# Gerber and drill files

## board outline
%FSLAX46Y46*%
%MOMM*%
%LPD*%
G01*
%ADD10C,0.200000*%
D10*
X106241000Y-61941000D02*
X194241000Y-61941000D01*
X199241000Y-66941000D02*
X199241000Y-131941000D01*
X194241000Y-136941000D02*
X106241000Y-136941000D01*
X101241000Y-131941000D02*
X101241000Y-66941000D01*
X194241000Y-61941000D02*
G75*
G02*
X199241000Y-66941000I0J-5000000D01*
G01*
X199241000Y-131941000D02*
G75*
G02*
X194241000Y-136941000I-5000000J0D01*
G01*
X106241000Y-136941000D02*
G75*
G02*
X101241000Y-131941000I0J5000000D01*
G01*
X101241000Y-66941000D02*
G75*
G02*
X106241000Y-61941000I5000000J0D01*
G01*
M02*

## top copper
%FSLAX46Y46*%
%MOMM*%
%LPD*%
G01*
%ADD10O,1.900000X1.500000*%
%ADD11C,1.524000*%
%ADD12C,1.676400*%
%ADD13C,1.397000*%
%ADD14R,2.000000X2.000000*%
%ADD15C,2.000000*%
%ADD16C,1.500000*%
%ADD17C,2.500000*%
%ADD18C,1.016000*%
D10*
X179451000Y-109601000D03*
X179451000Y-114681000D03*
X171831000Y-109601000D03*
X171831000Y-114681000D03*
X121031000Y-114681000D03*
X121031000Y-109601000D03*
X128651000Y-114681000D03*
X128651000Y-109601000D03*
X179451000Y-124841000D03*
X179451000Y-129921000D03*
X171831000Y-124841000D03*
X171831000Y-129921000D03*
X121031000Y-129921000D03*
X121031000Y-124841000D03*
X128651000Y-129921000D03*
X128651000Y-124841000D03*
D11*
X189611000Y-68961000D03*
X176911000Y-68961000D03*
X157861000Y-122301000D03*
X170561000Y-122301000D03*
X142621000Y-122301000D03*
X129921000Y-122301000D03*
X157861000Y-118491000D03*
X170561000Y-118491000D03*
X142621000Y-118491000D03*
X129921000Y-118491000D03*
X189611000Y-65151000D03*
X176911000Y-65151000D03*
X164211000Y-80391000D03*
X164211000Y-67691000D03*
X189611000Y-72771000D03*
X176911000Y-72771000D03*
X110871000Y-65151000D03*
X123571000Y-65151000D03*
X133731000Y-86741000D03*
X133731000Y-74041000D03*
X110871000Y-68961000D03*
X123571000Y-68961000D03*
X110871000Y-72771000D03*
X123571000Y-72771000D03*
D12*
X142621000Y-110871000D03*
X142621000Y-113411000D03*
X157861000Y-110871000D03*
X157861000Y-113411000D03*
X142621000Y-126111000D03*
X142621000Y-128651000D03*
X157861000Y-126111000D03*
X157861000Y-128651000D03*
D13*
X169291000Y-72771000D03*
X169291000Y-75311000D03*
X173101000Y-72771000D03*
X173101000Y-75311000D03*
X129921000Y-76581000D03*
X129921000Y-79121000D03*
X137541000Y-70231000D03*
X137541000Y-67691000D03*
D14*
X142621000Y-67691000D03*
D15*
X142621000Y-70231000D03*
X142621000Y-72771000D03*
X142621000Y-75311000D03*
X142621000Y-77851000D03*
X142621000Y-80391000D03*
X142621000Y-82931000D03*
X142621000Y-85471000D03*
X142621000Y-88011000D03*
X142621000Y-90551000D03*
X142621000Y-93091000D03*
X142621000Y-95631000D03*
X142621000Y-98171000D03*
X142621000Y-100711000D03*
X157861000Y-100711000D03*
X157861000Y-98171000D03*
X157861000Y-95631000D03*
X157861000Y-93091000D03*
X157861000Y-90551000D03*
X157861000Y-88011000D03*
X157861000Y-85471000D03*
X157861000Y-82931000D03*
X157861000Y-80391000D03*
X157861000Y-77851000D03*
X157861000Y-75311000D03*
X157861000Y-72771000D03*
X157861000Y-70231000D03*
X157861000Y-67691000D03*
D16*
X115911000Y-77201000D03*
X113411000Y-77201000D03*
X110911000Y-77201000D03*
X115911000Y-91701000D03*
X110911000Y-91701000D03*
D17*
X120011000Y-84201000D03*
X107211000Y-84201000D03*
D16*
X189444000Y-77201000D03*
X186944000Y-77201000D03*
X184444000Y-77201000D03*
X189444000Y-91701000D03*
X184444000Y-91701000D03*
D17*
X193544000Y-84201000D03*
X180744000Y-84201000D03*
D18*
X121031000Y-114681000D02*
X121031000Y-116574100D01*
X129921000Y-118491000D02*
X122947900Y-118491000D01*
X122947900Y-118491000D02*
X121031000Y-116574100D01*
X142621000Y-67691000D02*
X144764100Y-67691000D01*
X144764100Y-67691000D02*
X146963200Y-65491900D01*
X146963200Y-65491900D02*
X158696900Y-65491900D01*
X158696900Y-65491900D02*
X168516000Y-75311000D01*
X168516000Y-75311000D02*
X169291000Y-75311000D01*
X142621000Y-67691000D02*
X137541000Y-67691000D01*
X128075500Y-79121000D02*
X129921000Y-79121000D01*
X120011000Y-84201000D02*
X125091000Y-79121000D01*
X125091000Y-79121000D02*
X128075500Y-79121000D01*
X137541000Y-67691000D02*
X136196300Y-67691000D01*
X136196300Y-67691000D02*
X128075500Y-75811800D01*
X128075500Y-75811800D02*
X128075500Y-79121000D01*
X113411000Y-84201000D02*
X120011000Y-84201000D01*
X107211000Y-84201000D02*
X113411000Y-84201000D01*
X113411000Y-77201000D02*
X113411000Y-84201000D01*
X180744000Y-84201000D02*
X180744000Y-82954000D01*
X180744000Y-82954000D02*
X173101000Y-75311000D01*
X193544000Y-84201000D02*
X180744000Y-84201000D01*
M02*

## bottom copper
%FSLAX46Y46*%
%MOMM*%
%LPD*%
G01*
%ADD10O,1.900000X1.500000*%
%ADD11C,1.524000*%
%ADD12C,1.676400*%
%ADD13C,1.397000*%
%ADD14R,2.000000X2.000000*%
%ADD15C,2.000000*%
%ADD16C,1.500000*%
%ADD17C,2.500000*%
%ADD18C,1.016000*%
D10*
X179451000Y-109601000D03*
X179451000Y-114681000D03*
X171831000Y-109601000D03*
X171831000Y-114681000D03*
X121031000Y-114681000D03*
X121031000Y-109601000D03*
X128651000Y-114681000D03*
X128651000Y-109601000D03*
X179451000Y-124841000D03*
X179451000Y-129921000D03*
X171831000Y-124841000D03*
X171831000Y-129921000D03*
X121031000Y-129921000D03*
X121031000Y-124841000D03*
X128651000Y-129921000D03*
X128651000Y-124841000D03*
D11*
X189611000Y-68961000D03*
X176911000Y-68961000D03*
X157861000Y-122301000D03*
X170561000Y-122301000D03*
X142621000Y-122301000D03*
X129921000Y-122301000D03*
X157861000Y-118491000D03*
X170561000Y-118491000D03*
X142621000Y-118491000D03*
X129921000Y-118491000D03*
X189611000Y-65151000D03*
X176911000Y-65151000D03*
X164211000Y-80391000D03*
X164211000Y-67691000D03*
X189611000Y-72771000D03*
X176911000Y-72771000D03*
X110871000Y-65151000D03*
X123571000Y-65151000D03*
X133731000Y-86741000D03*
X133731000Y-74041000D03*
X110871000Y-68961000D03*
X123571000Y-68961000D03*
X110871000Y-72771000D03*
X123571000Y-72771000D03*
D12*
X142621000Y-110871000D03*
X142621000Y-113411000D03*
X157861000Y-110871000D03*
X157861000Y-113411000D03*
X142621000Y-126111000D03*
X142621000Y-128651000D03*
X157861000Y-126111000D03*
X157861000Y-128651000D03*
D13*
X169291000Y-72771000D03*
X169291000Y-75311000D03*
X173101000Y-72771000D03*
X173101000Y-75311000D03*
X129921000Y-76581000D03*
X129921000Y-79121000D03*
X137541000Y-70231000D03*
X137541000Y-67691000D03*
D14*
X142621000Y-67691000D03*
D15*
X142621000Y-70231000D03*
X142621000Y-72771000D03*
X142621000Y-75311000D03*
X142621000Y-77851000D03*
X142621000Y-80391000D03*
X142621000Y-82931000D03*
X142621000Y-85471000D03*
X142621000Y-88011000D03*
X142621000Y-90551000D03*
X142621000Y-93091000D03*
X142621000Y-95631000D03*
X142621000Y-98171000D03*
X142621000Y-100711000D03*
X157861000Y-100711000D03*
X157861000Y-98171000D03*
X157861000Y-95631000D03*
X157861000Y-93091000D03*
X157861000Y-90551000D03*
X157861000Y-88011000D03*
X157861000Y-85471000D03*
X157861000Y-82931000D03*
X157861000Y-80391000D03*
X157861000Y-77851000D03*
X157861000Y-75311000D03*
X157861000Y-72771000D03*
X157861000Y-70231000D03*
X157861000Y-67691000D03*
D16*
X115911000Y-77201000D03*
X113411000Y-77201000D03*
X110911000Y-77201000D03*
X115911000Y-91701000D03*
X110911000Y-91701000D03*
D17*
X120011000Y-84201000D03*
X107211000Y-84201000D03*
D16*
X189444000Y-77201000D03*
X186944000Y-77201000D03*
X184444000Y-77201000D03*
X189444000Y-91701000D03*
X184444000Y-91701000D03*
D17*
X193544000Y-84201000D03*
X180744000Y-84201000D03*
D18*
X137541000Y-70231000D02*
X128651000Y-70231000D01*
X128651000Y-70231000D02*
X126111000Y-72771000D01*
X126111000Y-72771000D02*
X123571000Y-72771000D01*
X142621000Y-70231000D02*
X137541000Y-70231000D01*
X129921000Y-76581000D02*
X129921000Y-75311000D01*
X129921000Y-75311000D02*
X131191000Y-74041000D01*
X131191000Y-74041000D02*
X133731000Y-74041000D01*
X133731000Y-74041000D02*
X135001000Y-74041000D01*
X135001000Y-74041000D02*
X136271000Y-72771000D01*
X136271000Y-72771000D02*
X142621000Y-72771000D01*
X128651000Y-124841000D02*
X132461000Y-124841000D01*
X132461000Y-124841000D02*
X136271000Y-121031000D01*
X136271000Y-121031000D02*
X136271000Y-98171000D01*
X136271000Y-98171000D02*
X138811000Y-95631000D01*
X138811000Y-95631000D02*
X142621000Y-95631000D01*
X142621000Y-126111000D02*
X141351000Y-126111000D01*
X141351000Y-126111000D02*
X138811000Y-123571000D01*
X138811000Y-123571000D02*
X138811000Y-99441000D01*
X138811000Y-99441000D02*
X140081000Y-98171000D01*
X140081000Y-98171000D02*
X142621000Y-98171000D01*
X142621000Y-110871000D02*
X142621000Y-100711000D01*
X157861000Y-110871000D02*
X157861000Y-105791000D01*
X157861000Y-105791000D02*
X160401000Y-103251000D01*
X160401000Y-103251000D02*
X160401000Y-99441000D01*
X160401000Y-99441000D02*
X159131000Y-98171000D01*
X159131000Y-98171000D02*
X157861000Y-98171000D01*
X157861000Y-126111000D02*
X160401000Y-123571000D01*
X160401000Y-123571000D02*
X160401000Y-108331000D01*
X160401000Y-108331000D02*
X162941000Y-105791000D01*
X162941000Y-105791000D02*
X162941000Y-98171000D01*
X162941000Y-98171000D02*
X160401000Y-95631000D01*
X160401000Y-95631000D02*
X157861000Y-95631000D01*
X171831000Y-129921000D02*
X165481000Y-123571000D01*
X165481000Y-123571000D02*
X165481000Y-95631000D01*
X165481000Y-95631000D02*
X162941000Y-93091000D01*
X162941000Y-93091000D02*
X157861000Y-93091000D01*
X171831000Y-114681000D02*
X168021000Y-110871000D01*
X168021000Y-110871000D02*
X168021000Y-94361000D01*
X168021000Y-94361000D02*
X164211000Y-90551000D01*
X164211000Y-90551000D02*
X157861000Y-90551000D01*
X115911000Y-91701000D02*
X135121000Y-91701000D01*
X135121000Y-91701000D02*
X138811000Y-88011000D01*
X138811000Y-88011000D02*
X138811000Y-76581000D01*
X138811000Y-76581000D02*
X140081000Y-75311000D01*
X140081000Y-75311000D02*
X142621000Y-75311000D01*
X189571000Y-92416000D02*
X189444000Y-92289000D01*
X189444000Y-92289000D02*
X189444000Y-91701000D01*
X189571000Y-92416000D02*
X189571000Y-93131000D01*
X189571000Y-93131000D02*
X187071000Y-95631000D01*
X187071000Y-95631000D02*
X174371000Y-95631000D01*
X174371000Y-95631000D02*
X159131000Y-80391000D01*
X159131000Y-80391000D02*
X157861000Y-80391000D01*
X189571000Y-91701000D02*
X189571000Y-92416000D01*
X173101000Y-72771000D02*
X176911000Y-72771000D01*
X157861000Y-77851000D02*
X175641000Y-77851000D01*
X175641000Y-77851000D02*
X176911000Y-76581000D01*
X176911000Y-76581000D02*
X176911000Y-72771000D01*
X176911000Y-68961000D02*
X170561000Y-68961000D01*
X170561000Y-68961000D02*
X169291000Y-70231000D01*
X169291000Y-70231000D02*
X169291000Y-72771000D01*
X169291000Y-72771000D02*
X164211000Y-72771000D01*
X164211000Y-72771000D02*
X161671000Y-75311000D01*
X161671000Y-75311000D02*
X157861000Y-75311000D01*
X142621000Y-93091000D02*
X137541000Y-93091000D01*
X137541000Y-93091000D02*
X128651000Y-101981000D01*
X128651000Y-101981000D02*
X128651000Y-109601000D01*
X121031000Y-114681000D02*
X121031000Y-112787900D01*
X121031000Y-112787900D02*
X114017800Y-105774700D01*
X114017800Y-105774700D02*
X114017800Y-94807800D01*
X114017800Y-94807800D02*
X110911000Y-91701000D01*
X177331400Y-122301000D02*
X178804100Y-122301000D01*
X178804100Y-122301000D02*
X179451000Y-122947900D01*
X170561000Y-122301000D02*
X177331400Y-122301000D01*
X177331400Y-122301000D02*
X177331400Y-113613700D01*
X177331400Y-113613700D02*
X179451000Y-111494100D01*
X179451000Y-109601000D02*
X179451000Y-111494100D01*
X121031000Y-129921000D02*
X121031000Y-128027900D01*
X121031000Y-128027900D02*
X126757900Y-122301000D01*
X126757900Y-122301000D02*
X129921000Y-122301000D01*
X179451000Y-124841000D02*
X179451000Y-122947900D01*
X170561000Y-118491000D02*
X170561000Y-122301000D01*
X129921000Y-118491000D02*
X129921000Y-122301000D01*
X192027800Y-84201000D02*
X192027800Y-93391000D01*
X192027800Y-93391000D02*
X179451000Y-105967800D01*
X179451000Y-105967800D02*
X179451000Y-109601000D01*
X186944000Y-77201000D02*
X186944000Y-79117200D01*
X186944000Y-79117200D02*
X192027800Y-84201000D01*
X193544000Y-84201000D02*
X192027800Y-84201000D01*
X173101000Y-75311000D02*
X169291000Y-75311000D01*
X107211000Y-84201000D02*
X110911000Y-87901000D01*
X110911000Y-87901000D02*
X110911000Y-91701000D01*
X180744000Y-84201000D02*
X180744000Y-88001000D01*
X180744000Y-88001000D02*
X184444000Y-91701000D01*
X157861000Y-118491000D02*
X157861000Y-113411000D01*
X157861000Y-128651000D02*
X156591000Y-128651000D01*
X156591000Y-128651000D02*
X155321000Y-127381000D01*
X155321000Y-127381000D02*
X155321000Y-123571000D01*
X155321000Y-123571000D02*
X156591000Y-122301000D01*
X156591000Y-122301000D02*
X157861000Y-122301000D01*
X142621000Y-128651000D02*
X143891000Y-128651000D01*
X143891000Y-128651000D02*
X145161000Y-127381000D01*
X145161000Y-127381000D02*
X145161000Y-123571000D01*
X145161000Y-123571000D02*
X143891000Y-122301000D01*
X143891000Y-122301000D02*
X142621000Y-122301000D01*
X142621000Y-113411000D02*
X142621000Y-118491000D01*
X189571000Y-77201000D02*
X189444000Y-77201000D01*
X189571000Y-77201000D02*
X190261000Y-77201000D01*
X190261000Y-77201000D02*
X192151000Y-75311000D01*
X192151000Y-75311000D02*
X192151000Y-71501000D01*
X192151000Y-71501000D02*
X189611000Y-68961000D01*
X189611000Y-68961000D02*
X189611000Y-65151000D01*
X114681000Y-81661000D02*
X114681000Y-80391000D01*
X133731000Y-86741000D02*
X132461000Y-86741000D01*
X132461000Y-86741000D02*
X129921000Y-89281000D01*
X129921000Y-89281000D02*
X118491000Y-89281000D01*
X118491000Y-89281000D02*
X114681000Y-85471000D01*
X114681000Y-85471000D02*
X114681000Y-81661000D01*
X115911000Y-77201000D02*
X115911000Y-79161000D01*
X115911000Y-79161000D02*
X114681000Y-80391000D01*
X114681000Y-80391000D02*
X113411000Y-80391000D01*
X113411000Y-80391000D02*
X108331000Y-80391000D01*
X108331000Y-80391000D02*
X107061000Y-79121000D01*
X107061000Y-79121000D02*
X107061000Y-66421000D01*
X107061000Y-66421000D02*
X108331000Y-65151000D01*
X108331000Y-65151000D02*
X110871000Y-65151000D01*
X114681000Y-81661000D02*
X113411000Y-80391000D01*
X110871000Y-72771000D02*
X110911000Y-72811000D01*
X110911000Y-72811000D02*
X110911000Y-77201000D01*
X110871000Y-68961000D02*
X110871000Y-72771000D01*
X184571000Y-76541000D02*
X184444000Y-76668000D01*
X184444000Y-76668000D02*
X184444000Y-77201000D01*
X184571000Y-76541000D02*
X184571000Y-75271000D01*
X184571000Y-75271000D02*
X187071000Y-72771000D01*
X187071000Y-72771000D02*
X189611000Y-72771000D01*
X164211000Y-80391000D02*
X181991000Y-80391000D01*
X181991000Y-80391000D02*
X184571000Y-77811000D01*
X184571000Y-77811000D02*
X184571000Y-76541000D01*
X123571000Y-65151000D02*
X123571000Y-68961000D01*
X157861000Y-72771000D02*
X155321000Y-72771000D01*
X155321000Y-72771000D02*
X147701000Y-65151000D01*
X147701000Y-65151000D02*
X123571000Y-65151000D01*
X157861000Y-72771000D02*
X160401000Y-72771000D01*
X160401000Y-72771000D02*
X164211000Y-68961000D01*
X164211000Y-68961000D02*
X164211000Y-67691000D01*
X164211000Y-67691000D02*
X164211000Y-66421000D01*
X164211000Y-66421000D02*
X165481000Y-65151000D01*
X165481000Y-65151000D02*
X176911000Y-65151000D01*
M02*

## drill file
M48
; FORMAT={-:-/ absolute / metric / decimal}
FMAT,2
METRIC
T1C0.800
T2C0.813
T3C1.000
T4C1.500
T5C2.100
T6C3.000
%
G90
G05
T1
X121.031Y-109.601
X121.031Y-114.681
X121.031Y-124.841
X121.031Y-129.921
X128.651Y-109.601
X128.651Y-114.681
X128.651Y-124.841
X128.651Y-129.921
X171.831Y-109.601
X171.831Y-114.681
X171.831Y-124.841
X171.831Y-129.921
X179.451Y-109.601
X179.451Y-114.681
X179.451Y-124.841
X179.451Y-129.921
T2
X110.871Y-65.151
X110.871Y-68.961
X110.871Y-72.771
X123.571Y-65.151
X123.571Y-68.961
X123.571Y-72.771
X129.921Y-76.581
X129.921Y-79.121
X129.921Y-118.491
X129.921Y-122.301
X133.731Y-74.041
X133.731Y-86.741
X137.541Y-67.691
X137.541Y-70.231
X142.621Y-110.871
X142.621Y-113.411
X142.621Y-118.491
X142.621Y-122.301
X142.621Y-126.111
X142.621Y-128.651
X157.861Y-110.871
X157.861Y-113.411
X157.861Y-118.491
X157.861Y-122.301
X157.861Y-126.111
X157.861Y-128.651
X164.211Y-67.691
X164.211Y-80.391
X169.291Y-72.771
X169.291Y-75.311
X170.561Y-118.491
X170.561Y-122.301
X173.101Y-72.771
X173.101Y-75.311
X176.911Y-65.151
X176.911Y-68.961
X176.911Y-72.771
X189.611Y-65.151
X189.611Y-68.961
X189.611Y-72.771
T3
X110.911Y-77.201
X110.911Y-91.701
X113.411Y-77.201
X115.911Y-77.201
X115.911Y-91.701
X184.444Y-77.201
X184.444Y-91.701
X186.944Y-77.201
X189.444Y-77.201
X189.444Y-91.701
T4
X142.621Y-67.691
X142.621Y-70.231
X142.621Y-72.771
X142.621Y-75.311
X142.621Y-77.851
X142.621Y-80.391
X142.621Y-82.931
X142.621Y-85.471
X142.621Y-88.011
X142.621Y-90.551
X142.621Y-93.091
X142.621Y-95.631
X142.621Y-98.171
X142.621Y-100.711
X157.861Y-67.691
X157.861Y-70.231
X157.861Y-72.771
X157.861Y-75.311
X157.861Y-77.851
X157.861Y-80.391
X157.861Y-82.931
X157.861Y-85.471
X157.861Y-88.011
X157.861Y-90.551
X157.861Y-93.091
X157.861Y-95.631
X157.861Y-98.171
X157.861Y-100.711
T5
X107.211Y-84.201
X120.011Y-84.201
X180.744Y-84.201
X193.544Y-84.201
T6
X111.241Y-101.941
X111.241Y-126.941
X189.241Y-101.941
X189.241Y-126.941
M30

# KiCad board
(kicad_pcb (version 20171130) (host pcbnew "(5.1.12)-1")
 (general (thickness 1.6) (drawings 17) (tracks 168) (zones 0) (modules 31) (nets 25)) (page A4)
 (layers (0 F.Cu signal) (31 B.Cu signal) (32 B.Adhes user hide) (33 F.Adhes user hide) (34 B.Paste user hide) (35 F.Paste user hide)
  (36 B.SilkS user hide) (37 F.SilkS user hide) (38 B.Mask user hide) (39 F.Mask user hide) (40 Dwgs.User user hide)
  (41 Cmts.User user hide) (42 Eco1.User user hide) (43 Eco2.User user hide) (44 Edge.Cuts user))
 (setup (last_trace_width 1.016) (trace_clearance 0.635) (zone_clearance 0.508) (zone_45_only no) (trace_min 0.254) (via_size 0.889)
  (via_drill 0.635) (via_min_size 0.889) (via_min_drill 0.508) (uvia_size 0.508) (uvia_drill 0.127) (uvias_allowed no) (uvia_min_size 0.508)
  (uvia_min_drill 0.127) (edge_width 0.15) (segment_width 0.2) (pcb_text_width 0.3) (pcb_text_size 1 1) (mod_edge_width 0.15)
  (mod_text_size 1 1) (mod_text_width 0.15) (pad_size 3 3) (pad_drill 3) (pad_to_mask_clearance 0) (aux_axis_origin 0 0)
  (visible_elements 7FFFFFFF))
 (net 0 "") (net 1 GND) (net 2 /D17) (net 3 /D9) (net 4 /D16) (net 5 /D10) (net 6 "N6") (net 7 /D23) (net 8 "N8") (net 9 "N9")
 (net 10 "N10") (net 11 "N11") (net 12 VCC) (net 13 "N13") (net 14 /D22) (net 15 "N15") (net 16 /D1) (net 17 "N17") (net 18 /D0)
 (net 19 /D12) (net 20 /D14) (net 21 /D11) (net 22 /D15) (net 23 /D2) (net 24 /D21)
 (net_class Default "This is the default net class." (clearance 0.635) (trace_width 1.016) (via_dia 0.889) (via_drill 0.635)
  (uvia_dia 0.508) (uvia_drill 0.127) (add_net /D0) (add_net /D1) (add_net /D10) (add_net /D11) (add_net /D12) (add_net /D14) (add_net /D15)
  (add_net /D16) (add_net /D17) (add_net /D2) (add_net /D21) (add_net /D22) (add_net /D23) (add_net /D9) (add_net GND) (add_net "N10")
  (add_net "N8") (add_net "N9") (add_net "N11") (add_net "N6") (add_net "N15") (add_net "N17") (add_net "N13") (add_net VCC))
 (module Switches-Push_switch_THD (layer F.Cu) (at 175.641 112.141 180)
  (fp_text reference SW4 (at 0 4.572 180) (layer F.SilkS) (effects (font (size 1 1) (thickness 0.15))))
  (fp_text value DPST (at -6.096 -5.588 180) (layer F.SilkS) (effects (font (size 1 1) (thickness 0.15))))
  (pad 2 thru_hole oval (at -3.81 2.54 180) (size 1.9 1.5) (drill 0.8) (layers *.Cu *.Mask F.SilkS) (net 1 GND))
  (pad 1 thru_hole oval (at -3.81 -2.54 180) (size 1.9 1.5) (drill 0.8) (layers *.Cu *.Mask F.SilkS))
  (pad 4 thru_hole oval (at 3.81 2.54 180) (size 1.9 1.5) (drill 0.8) (layers *.Cu *.Mask F.SilkS))
  (pad 3 thru_hole oval (at 3.81 -2.54 180) (size 1.9 1.5) (drill 0.8) (layers *.Cu *.Mask F.SilkS) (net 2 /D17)))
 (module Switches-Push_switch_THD (layer F.Cu) (at 124.841 112.141)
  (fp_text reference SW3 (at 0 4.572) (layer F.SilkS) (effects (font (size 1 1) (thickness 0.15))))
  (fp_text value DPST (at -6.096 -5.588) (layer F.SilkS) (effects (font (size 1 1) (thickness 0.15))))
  (pad 2 thru_hole oval (at -3.81 2.54) (size 1.9 1.5) (drill 0.8) (layers *.Cu *.Mask F.SilkS) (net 1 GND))
  (pad 1 thru_hole oval (at -3.81 -2.54) (size 1.9 1.5) (drill 0.8) (layers *.Cu *.Mask F.SilkS))
  (pad 4 thru_hole oval (at 3.81 2.54) (size 1.9 1.5) (drill 0.8) (layers *.Cu *.Mask F.SilkS))
  (pad 3 thru_hole oval (at 3.81 -2.54) (size 1.9 1.5) (drill 0.8) (layers *.Cu *.Mask F.SilkS) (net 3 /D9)))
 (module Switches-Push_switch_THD (layer F.Cu) (at 175.641 127.381 180)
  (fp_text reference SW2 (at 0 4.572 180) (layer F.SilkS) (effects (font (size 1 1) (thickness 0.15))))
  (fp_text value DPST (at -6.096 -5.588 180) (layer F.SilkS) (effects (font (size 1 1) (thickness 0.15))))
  (pad 2 thru_hole oval (at -3.81 2.54 180) (size 1.9 1.5) (drill 0.8) (layers *.Cu *.Mask F.SilkS) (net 1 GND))
  (pad 1 thru_hole oval (at -3.81 -2.54 180) (size 1.9 1.5) (drill 0.8) (layers *.Cu *.Mask F.SilkS))
  (pad 4 thru_hole oval (at 3.81 2.54 180) (size 1.9 1.5) (drill 0.8) (layers *.Cu *.Mask F.SilkS))
  (pad 3 thru_hole oval (at 3.81 -2.54 180) (size 1.9 1.5) (drill 0.8) (layers *.Cu *.Mask F.SilkS) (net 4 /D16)))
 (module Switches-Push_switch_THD (layer F.Cu) (at 124.841 127.381)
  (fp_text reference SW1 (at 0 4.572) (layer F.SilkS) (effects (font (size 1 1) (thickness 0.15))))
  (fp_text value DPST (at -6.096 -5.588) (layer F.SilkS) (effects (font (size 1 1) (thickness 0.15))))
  (pad 2 thru_hole oval (at -3.81 2.54) (size 1.9 1.5) (drill 0.8) (layers *.Cu *.Mask F.SilkS) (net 1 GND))
  (pad 1 thru_hole oval (at -3.81 -2.54) (size 1.9 1.5) (drill 0.8) (layers *.Cu *.Mask F.SilkS))
  (pad 4 thru_hole oval (at 3.81 2.54) (size 1.9 1.5) (drill 0.8) (layers *.Cu *.Mask F.SilkS))
  (pad 3 thru_hole oval (at 3.81 -2.54) (size 1.9 1.5) (drill 0.8) (layers *.Cu *.Mask F.SilkS) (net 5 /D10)))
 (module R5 (layer F.Cu) (at 183.261 68.961 180) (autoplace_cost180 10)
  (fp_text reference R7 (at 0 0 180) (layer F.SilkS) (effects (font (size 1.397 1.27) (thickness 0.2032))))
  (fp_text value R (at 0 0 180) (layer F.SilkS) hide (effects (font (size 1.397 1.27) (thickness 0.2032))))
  (pad 1 thru_hole circle (at -6.35 0 180) (size 1.524 1.524) (drill 0.8128) (layers *.Cu *.Mask F.SilkS) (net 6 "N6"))
  (pad 2 thru_hole circle (at 6.35 0 180) (size 1.524 1.524) (drill 0.8128) (layers *.Cu *.Mask F.SilkS) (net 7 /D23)))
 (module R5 (layer F.Cu) (at 164.211 122.301) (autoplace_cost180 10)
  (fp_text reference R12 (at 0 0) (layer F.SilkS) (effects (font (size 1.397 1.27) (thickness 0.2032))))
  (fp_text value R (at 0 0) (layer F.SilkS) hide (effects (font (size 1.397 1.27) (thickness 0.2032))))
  (pad 1 thru_hole circle (at -6.35 0) (size 1.524 1.524) (drill 0.8128) (layers *.Cu *.Mask F.SilkS) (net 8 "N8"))
  (pad 2 thru_hole circle (at 6.35 0) (size 1.524 1.524) (drill 0.8128) (layers *.Cu *.Mask F.SilkS) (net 1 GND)))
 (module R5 (layer F.Cu) (at 136.271 122.301 180) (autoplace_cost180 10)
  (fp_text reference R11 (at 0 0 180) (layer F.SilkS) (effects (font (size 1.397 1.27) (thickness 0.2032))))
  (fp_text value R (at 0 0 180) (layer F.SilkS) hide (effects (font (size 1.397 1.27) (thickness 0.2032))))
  (pad 1 thru_hole circle (at -6.35 0 180) (size 1.524 1.524) (drill 0.8128) (layers *.Cu *.Mask F.SilkS) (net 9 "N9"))
  (pad 2 thru_hole circle (at 6.35 0 180) (size 1.524 1.524) (drill 0.8128) (layers *.Cu *.Mask F.SilkS) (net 1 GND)))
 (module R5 (layer F.Cu) (at 164.211 118.491) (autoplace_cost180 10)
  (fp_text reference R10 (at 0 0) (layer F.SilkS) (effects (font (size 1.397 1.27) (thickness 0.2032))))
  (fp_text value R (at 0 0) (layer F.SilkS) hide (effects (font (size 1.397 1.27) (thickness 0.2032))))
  (pad 1 thru_hole circle (at -6.35 0) (size 1.524 1.524) (drill 0.8128) (layers *.Cu *.Mask F.SilkS) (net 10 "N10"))
  (pad 2 thru_hole circle (at 6.35 0) (size 1.524 1.524) (drill 0.8128) (layers *.Cu *.Mask F.SilkS) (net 1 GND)))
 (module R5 (layer F.Cu) (at 136.271 118.491 180) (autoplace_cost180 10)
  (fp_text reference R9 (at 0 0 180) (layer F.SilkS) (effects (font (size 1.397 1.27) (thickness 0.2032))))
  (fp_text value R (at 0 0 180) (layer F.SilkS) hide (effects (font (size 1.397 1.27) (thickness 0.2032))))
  (pad 1 thru_hole circle (at -6.35 0 180) (size 1.524 1.524) (drill 0.8128) (layers *.Cu *.Mask F.SilkS) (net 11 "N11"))
  (pad 2 thru_hole circle (at 6.35 0 180) (size 1.524 1.524) (drill 0.8128) (layers *.Cu *.Mask F.SilkS) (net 1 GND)))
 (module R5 (layer F.Cu) (at 183.261 65.151 180) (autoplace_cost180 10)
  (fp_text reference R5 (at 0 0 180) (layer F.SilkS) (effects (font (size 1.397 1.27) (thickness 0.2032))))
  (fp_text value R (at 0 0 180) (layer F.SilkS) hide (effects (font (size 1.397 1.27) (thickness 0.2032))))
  (pad 1 thru_hole circle (at -6.35 0 180) (size 1.524 1.524) (drill 0.8128) (layers *.Cu *.Mask F.SilkS) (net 6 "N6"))
  (pad 2 thru_hole circle (at 6.35 0 180) (size 1.524 1.524) (drill 0.8128) (layers *.Cu *.Mask F.SilkS) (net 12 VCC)))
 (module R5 (layer F.Cu) (at 164.211 74.041 90) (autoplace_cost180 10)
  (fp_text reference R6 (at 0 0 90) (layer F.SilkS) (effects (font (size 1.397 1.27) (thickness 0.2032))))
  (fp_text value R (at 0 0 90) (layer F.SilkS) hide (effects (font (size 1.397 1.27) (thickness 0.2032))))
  (pad 1 thru_hole circle (at -6.35 0 90) (size 1.524 1.524) (drill 0.8128) (layers *.Cu *.Mask F.SilkS) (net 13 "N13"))
  (pad 2 thru_hole circle (at 6.35 0 90) (size 1.524 1.524) (drill 0.8128) (layers *.Cu *.Mask F.SilkS) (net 12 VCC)))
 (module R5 (layer F.Cu) (at 183.261 72.771 180) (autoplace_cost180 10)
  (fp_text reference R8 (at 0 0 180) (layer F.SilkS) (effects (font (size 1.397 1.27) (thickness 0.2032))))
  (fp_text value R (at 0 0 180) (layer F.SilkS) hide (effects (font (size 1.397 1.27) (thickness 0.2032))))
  (pad 1 thru_hole circle (at -6.35 0 180) (size 1.524 1.524) (drill 0.8128) (layers *.Cu *.Mask F.SilkS) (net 13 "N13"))
  (pad 2 thru_hole circle (at 6.35 0 180) (size 1.524 1.524) (drill 0.8128) (layers *.Cu *.Mask F.SilkS) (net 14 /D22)))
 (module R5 (layer F.Cu) (at 117.221 65.151) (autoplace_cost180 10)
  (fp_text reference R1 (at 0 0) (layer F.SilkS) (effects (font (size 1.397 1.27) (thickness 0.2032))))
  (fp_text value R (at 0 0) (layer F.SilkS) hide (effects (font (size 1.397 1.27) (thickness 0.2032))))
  (pad 1 thru_hole circle (at -6.35 0) (size 1.524 1.524) (drill 0.8128) (layers *.Cu *.Mask F.SilkS) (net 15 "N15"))
  (pad 2 thru_hole circle (at 6.35 0) (size 1.524 1.524) (drill 0.8128) (layers *.Cu *.Mask F.SilkS) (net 12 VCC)))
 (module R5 (layer F.Cu) (at 133.731 80.391 90) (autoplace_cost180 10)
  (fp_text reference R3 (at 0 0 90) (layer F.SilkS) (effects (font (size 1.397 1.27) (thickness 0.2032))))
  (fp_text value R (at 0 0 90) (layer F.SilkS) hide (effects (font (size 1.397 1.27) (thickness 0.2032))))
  (pad 1 thru_hole circle (at -6.35 0 90) (size 1.524 1.524) (drill 0.8128) (layers *.Cu *.Mask F.SilkS) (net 15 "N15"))
  (pad 2 thru_hole circle (at 6.35 0 90) (size 1.524 1.524) (drill 0.8128) (layers *.Cu *.Mask F.SilkS) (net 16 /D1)))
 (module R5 (layer F.Cu) (at 117.221 68.961) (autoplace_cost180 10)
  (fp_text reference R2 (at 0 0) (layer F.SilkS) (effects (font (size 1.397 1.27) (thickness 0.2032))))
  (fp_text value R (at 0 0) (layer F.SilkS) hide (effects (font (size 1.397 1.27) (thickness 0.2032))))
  (pad 1 thru_hole circle (at -6.35 0) (size 1.524 1.524) (drill 0.8128) (layers *.Cu *.Mask F.SilkS) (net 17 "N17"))
  (pad 2 thru_hole circle (at 6.35 0) (size 1.524 1.524) (drill 0.8128) (layers *.Cu *.Mask F.SilkS) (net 12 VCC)))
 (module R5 (layer F.Cu) (at 117.221 72.771) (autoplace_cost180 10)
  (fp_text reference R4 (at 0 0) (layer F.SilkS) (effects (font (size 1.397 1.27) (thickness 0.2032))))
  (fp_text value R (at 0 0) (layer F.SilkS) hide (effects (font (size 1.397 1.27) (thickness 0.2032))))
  (pad 1 thru_hole circle (at -6.35 0) (size 1.524 1.524) (drill 0.8128) (layers *.Cu *.Mask F.SilkS) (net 17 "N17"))
  (pad 2 thru_hole circle (at 6.35 0) (size 1.524 1.524) (drill 0.8128) (layers *.Cu *.Mask F.SilkS) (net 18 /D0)))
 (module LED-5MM (layer F.Cu) (at 142.621 112.141 270)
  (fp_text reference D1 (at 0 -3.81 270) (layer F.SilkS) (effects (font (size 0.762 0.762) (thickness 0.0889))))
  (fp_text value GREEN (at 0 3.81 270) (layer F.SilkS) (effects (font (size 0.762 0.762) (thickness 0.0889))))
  (pad 1 thru_hole circle (at -1.27 0 270) (size 1.6764 1.6764) (drill 0.8128) (layers *.Cu *.Mask F.SilkS) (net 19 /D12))
  (pad 2 thru_hole circle (at 1.27 0 270) (size 1.6764 1.6764) (drill 0.8128) (layers *.Cu *.Mask F.SilkS) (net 11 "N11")))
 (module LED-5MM (layer F.Cu) (at 157.861 112.141 270)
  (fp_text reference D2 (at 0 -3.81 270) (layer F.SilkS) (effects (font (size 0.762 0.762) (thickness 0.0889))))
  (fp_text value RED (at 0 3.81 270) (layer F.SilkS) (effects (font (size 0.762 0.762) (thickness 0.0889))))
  (pad 1 thru_hole circle (at -1.27 0 270) (size 1.6764 1.6764) (drill 0.8128) (layers *.Cu *.Mask F.SilkS) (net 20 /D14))
  (pad 2 thru_hole circle (at 1.27 0 270) (size 1.6764 1.6764) (drill 0.8128) (layers *.Cu *.Mask F.SilkS) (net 10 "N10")))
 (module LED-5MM (layer F.Cu) (at 142.621 127.381 270)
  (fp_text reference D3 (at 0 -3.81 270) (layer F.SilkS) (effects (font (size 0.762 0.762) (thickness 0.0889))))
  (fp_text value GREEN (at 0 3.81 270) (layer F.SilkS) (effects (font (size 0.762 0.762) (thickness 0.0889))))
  (pad 1 thru_hole circle (at -1.27 0 270) (size 1.6764 1.6764) (drill 0.8128) (layers *.Cu *.Mask F.SilkS) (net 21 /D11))
  (pad 2 thru_hole circle (at 1.27 0 270) (size 1.6764 1.6764) (drill 0.8128) (layers *.Cu *.Mask F.SilkS) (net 9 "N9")))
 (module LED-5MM (layer F.Cu) (at 157.861 127.381 270)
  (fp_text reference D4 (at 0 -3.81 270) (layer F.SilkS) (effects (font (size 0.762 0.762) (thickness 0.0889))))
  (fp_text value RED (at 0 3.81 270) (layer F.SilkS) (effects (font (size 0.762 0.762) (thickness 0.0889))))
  (pad 1 thru_hole circle (at -1.27 0 270) (size 1.6764 1.6764) (drill 0.8128) (layers *.Cu *.Mask F.SilkS) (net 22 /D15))
  (pad 2 thru_hole circle (at 1.27 0 270) (size 1.6764 1.6764) (drill 0.8128) (layers *.Cu *.Mask F.SilkS) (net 8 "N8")))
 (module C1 (layer F.Cu) (at 169.291 74.041 270)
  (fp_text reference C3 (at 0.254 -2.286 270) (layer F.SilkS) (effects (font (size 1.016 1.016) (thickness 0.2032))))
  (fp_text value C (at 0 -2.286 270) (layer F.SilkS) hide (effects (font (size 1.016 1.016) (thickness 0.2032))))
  (pad 1 thru_hole circle (at -1.27 0 270) (size 1.397 1.397) (drill 0.8128) (layers *.Cu *.Mask F.SilkS) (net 7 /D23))
  (pad 2 thru_hole circle (at 1.27 0 270) (size 1.397 1.397) (drill 0.8128) (layers *.Cu *.Mask F.SilkS) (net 1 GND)))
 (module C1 (layer F.Cu) (at 173.101 74.041 270)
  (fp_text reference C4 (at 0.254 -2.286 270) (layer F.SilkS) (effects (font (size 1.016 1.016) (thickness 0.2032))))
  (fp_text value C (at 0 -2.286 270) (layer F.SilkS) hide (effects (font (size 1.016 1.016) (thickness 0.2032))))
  (pad 1 thru_hole circle (at -1.27 0 270) (size 1.397 1.397) (drill 0.8128) (layers *.Cu *.Mask F.SilkS) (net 14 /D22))
  (pad 2 thru_hole circle (at 1.27 0 270) (size 1.397 1.397) (drill 0.8128) (layers *.Cu *.Mask F.SilkS) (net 1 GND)))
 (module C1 (layer F.Cu) (at 129.921 77.851 270)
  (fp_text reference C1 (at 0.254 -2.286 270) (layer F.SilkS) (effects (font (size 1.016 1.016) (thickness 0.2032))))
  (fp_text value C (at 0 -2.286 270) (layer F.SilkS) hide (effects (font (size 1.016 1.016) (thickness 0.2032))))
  (pad 1 thru_hole circle (at -1.27 0 270) (size 1.397 1.397) (drill 0.8128) (layers *.Cu *.Mask F.SilkS) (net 16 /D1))
  (pad 2 thru_hole circle (at 1.27 0 270) (size 1.397 1.397) (drill 0.8128) (layers *.Cu *.Mask F.SilkS) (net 1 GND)))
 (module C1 (layer F.Cu) (at 137.541 68.961 90)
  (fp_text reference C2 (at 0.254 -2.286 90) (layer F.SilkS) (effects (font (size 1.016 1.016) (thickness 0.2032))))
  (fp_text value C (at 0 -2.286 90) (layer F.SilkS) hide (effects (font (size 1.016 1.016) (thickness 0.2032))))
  (pad 1 thru_hole circle (at -1.27 0 90) (size 1.397 1.397) (drill 0.8128) (layers *.Cu *.Mask F.SilkS) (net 18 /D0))
  (pad 2 thru_hole circle (at 1.27 0 90) (size 1.397 1.397) (drill 0.8128) (layers *.Cu *.Mask F.SilkS) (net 1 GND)))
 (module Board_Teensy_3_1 (layer F.Cu) (at 150.241 85.471)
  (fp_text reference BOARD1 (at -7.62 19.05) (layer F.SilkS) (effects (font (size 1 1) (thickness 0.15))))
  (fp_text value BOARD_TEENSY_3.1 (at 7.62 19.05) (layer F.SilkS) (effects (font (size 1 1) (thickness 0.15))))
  (pad 1 thru_hole rect (at -7.62 -17.78) (size 2 2) (drill 1.5) (layers *.Cu *.Mask F.SilkS) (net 1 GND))
  (pad 2 thru_hole circle (at -7.62 -15.24) (size 2 2) (drill 1.5) (layers *.Cu *.Mask F.SilkS) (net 18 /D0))
  (pad 3 thru_hole circle (at -7.62 -12.7) (size 2 2) (drill 1.5) (layers *.Cu *.Mask F.SilkS) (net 16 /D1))
  (pad 4 thru_hole circle (at -7.62 -10.16) (size 2 2) (drill 1.5) (layers *.Cu *.Mask F.SilkS) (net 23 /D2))
  (pad 5 thru_hole circle (at -7.62 -7.62) (size 2 2) (drill 1.5) (layers *.Cu *.Mask F.SilkS))
  (pad 6 thru_hole circle (at -7.62 -5.08) (size 2 2) (drill 1.5) (layers *.Cu *.Mask F.SilkS))
  (pad 7 thru_hole circle (at -7.62 -2.54) (size 2 2) (drill 1.5) (layers *.Cu *.Mask F.SilkS))
  (pad 8 thru_hole circle (at -7.62 0) (size 2 2) (drill 1.5) (layers *.Cu *.Mask F.SilkS))
  (pad 9 thru_hole circle (at -7.62 2.54) (size 2 2) (drill 1.5) (layers *.Cu *.Mask F.SilkS))
  (pad 10 thru_hole circle (at -7.62 5.08) (size 2 2) (drill 1.5) (layers *.Cu *.Mask F.SilkS))
  (pad 11 thru_hole circle (at -7.62 7.62) (size 2 2) (drill 1.5) (layers *.Cu *.Mask F.SilkS) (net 3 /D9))
  (pad 12 thru_hole circle (at -7.62 10.16) (size 2 2) (drill 1.5) (layers *.Cu *.Mask F.SilkS) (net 5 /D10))
  (pad 13 thru_hole circle (at -7.62 12.7) (size 2 2) (drill 1.5) (layers *.Cu *.Mask F.SilkS) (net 21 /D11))
  (pad 14 thru_hole circle (at -7.62 15.24) (size 2 2) (drill 1.5) (layers *.Cu *.Mask F.SilkS) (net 19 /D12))
  (pad 15 thru_hole circle (at 7.62 15.24) (size 2 2) (drill 1.5) (layers *.Cu *.Mask F.SilkS))
  (pad 16 thru_hole circle (at 7.62 12.7) (size 2 2) (drill 1.5) (layers *.Cu *.Mask F.SilkS) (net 20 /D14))
  (pad 17 thru_hole circle (at 7.62 10.16) (size 2 2) (drill 1.5) (layers *.Cu *.Mask F.SilkS) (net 22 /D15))
  (pad 18 thru_hole circle (at 7.62 7.62) (size 2 2) (drill 1.5) (layers *.Cu *.Mask F.SilkS) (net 4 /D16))
  (pad 19 thru_hole circle (at 7.62 5.08) (size 2 2) (drill 1.5) (layers *.Cu *.Mask F.SilkS) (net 2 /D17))
  (pad 20 thru_hole circle (at 7.62 2.54) (size 2 2) (drill 1.5) (layers *.Cu *.Mask F.SilkS))
  (pad 21 thru_hole circle (at 7.62 0) (size 2 2) (drill 1.5) (layers *.Cu *.Mask F.SilkS))
  (pad 22 thru_hole circle (at 7.62 -2.54) (size 2 2) (drill 1.5) (layers *.Cu *.Mask F.SilkS))
  (pad 23 thru_hole circle (at 7.62 -5.08) (size 2 2) (drill 1.5) (layers *.Cu *.Mask F.SilkS) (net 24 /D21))
  (pad 24 thru_hole circle (at 7.62 -7.62) (size 2 2) (drill 1.5) (layers *.Cu *.Mask F.SilkS) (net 14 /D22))
  (pad 25 thru_hole circle (at 7.62 -10.16) (size 2 2) (drill 1.5) (layers *.Cu *.Mask F.SilkS) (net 7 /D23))
  (pad 26 thru_hole circle (at 7.62 -12.7) (size 2 2) (drill 1.5) (layers *.Cu *.Mask F.SilkS) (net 12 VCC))
  (pad 27 thru_hole circle (at 7.62 -15.24) (size 2 2) (drill 1.5) (layers *.Cu *.Mask F.SilkS))
  (pad 28 thru_hole circle (at 7.62 -17.78) (size 2 2) (drill 1.5) (layers *.Cu *.Mask F.SilkS)))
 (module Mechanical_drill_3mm (layer F.Cu) (at 107.95 130.81)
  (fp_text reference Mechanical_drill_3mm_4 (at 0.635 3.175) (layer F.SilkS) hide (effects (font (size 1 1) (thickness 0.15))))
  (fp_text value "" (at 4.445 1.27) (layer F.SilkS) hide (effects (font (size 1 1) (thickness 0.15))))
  (pad "" np_thru_hole circle (at 3.291 -3.869) (size 3 3) (drill 3) (layers *.Cu *.Mask)))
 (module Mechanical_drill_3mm (layer F.Cu) (at 193.04 130.81)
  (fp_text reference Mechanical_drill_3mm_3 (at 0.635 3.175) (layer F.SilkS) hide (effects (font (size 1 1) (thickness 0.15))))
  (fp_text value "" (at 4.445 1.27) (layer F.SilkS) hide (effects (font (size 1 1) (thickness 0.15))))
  (pad "" np_thru_hole circle (at -3.799 -3.869) (size 3 3) (drill 3) (layers *.Cu *.Mask)))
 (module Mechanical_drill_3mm (layer F.Cu) (at 191.77 102.87)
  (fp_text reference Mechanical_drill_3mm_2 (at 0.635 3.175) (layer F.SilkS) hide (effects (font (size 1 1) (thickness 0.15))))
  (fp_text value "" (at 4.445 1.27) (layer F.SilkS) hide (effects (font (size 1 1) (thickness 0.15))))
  (pad "" np_thru_hole circle (at -2.529 -0.929) (size 3 3) (drill 3) (layers *.Cu *.Mask)))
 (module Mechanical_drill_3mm (layer F.Cu) (at 107.95 101.6)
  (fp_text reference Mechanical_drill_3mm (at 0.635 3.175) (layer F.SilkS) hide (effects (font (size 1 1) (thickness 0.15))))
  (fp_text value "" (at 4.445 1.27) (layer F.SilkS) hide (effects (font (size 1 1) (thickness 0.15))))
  (pad "" np_thru_hole circle (at 3.291 0.341) (size 3 3) (drill 3) (layers *.Cu *.Mask)))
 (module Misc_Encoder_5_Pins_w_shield (layer F.Cu) (at 113.411 84.201 270)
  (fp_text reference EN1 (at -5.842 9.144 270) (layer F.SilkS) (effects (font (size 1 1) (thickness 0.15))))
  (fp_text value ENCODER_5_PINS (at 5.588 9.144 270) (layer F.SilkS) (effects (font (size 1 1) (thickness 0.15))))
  (pad 1 thru_hole circle (at -7 -2.5 270) (size 1.5 1.5) (drill 1) (layers *.Cu *.Mask F.SilkS) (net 15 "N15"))
  (pad 2 thru_hole circle (at -7 0 270) (size 1.5 1.5) (drill 1) (layers *.Cu *.Mask F.SilkS) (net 1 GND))
  (pad 3 thru_hole circle (at -7 2.5 270) (size 1.5 1.5) (drill 1) (layers *.Cu *.Mask F.SilkS) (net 17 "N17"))
  (pad 4 thru_hole circle (at 7.5 -2.5 270) (size 1.5 1.5) (drill 1) (layers *.Cu *.Mask F.SilkS) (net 23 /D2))
  (pad 5 thru_hole circle (at 7.5 2.5 270) (size 1.5 1.5) (drill 1) (layers *.Cu *.Mask F.SilkS) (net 1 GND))
  (pad SHLD thru_hole circle (at 0 -6.6 270) (size 2.5 2.5) (drill 2.1) (layers *.Cu *.Mask F.SilkS) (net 1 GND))
  (pad SHLD thru_hole circle (at 0 6.2 270) (size 2.5 2.5) (drill 2.1) (layers *.Cu *.Mask F.SilkS) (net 1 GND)))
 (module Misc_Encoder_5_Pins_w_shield (layer F.Cu) (at 186.944 84.201 270)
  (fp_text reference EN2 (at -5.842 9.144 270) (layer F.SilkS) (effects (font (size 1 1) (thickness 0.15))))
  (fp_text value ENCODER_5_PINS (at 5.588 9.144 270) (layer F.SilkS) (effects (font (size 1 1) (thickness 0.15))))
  (pad 1 thru_hole circle (at -7 -2.5 270) (size 1.5 1.5) (drill 1) (layers *.Cu *.Mask F.SilkS) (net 6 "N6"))
  (pad 2 thru_hole circle (at -7 0 270) (size 1.5 1.5) (drill 1) (layers *.Cu *.Mask F.SilkS) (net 1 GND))
  (pad 3 thru_hole circle (at -7 2.5 270) (size 1.5 1.5) (drill 1) (layers *.Cu *.Mask F.SilkS) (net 13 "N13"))
  (pad 4 thru_hole circle (at 7.5 -2.5 270) (size 1.5 1.5) (drill 1) (layers *.Cu *.Mask F.SilkS) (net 24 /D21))
  (pad 5 thru_hole circle (at 7.5 2.5 270) (size 1.5 1.5) (drill 1) (layers *.Cu *.Mask F.SilkS) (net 1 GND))
  (pad SHLD thru_hole circle (at 0 -6.6 270) (size 2.5 2.5) (drill 2.1) (layers *.Cu *.Mask F.SilkS) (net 1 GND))
  (pad SHLD thru_hole circle (at 0 6.2 270) (size 2.5 2.5) (drill 2.1) (layers *.Cu *.Mask F.SilkS) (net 1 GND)))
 (gr_line (start 106.241 61.941) (end 194.241 61.941) (angle 90) (layer Edge.Cuts) (width 0.2))
 (gr_line (start 199.241 66.941) (end 199.241 131.941) (angle 90) (layer Edge.Cuts) (width 0.2))
 (gr_line (start 194.241 136.941) (end 106.241 136.941) (angle 90) (layer Edge.Cuts) (width 0.2))
 (gr_line (start 101.241 131.941) (end 101.241 66.941) (angle 90) (layer Edge.Cuts) (width 0.2))
 (gr_arc (start 194.241 66.941) (end 194.241 61.941) (angle 90) (layer Edge.Cuts) (width 0.2))
 (gr_arc (start 194.241 131.941) (end 199.241 131.941) (angle 90) (layer Edge.Cuts) (width 0.2))
 (gr_arc (start 106.241 131.941) (end 106.241 136.941) (angle 90) (layer Edge.Cuts) (width 0.2))
 (gr_arc (start 106.241 66.941) (end 101.241 66.941) (angle 90) (layer Edge.Cuts) (width 0.2))
 (segment (start 137.541 70.231) (end 128.651 70.231) (width 1.016) (layer B.Cu) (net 18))
 (segment (start 128.651 70.231) (end 126.111 72.771) (width 1.016) (layer B.Cu) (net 18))
 (segment (start 126.111 72.771) (end 123.571 72.771) (width 1.016) (layer B.Cu) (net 18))
 (segment (start 142.621 70.231) (end 137.541 70.231) (width 1.016) (layer B.Cu) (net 18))
 (segment (start 129.921 76.581) (end 129.921 75.311) (width 1.016) (layer B.Cu) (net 16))
 (segment (start 129.921 75.311) (end 131.191 74.041) (width 1.016) (layer B.Cu) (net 16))
 (segment (start 131.191 74.041) (end 133.731 74.041) (width 1.016) (layer B.Cu) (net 16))
 (segment (start 133.731 74.041) (end 135.001 74.041) (width 1.016) (layer B.Cu) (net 16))
 (segment (start 135.001 74.041) (end 136.271 72.771) (width 1.016) (layer B.Cu) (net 16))
 (segment (start 136.271 72.771) (end 142.621 72.771) (width 1.016) (layer B.Cu) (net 16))
 (segment (start 128.651 124.841) (end 132.461 124.841) (width 1.016) (layer B.Cu) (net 5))
 (segment (start 132.461 124.841) (end 136.271 121.031) (width 1.016) (layer B.Cu) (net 5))
 (segment (start 136.271 121.031) (end 136.271 98.171) (width 1.016) (layer B.Cu) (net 5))
 (segment (start 136.271 98.171) (end 138.811 95.631) (width 1.016) (layer B.Cu) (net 5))
 (segment (start 138.811 95.631) (end 142.621 95.631) (width 1.016) (layer B.Cu) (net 5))
 (segment (start 142.621 126.111) (end 141.351 126.111) (width 1.016) (layer B.Cu) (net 21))
 (segment (start 141.351 126.111) (end 138.811 123.571) (width 1.016) (layer B.Cu) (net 21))
 (segment (start 138.811 123.571) (end 138.811 99.441) (width 1.016) (layer B.Cu) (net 21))
 (segment (start 138.811 99.441) (end 140.081 98.171) (width 1.016) (layer B.Cu) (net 21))
 (segment (start 140.081 98.171) (end 142.621 98.171) (width 1.016) (layer B.Cu) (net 21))
 (segment (start 142.621 110.871) (end 142.621 100.711) (width 1.016) (layer B.Cu) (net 19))
 (segment (start 157.861 110.871) (end 157.861 105.791) (width 1.016) (layer B.Cu) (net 20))
 (segment (start 157.861 105.791) (end 160.401 103.251) (width 1.016) (layer B.Cu) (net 20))
 (segment (start 160.401 103.251) (end 160.401 99.441) (width 1.016) (layer B.Cu) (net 20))
 (segment (start 160.401 99.441) (end 159.131 98.171) (width 1.016) (layer B.Cu) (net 20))
 (segment (start 159.131 98.171) (end 157.861 98.171) (width 1.016) (layer B.Cu) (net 20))
 (segment (start 157.861 126.111) (end 160.401 123.571) (width 1.016) (layer B.Cu) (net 22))
 (segment (start 160.401 123.571) (end 160.401 108.331) (width 1.016) (layer B.Cu) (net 22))
 (segment (start 160.401 108.331) (end 162.941 105.791) (width 1.016) (layer B.Cu) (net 22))
 (segment (start 162.941 105.791) (end 162.941 98.171) (width 1.016) (layer B.Cu) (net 22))
 (segment (start 162.941 98.171) (end 160.401 95.631) (width 1.016) (layer B.Cu) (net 22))
 (segment (start 160.401 95.631) (end 157.861 95.631) (width 1.016) (layer B.Cu) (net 22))
 (segment (start 171.831 129.921) (end 165.481 123.571) (width 1.016) (layer B.Cu) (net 4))
 (segment (start 165.481 123.571) (end 165.481 95.631) (width 1.016) (layer B.Cu) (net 4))
 (segment (start 165.481 95.631) (end 162.941 93.091) (width 1.016) (layer B.Cu) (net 4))
 (segment (start 162.941 93.091) (end 157.861 93.091) (width 1.016) (layer B.Cu) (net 4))
 (segment (start 171.831 114.681) (end 168.021 110.871) (width 1.016) (layer B.Cu) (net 2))
 (segment (start 168.021 110.871) (end 168.021 94.361) (width 1.016) (layer B.Cu) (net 2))
 (segment (start 168.021 94.361) (end 164.211 90.551) (width 1.016) (layer B.Cu) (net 2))
 (segment (start 164.211 90.551) (end 157.861 90.551) (width 1.016) (layer B.Cu) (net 2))
 (segment (start 115.911 91.701) (end 135.121 91.701) (width 1.016) (layer B.Cu) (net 23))
 (segment (start 135.121 91.701) (end 138.811 88.011) (width 1.016) (layer B.Cu) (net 23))
 (segment (start 138.811 88.011) (end 138.811 76.581) (width 1.016) (layer B.Cu) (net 23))
 (segment (start 138.811 76.581) (end 140.081 75.311) (width 1.016) (layer B.Cu) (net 23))
 (segment (start 140.081 75.311) (end 142.621 75.311) (width 1.016) (layer B.Cu) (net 23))
 (segment (start 189.571 92.416) (end 189.444 92.289) (width 1.016) (layer B.Cu) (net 24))
 (segment (start 189.444 92.289) (end 189.444 91.701) (width 1.016) (layer B.Cu) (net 24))
 (segment (start 189.571 92.416) (end 189.571 93.131) (width 1.016) (layer B.Cu) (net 24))
 (segment (start 189.571 93.131) (end 187.071 95.631) (width 1.016) (layer B.Cu) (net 24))
 (segment (start 187.071 95.631) (end 174.371 95.631) (width 1.016) (layer B.Cu) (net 24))
 (segment (start 174.371 95.631) (end 159.131 80.391) (width 1.016) (layer B.Cu) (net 24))
 (segment (start 159.131 80.391) (end 157.861 80.391) (width 1.016) (layer B.Cu) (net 24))
 (segment (start 189.571 91.701) (end 189.571 92.416) (width 1.016) (layer B.Cu) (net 24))
 (segment (start 173.101 72.771) (end 176.911 72.771) (width 1.016) (layer B.Cu) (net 14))
 (segment (start 157.861 77.851) (end 175.641 77.851) (width 1.016) (layer B.Cu) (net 14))
 (segment (start 175.641 77.851) (end 176.911 76.581) (width 1.016) (layer B.Cu) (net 14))
 (segment (start 176.911 76.581) (end 176.911 72.771) (width 1.016) (layer B.Cu) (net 14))
 (segment (start 176.911 68.961) (end 170.561 68.961) (width 1.016) (layer B.Cu) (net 7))
 (segment (start 170.561 68.961) (end 169.291 70.231) (width 1.016) (layer B.Cu) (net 7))
 (segment (start 169.291 70.231) (end 169.291 72.771) (width 1.016) (layer B.Cu) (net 7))
 (segment (start 169.291 72.771) (end 164.211 72.771) (width 1.016) (layer B.Cu) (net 7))
 (segment (start 164.211 72.771) (end 161.671 75.311) (width 1.016) (layer B.Cu) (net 7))
 (segment (start 161.671 75.311) (end 157.861 75.311) (width 1.016) (layer B.Cu) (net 7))
 (segment (start 142.621 93.091) (end 137.541 93.091) (width 1.016) (layer B.Cu) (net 3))
 (segment (start 137.541 93.091) (end 128.651 101.981) (width 1.016) (layer B.Cu) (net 3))
 (segment (start 128.651 101.981) (end 128.651 109.601) (width 1.016) (layer B.Cu) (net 3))
 (segment (start 121.031 114.681) (end 121.031 112.7879) (width 1.016) (layer B.Cu) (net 1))
 (segment (start 121.031 112.7879) (end 114.0178 105.7747) (width 1.016) (layer B.Cu) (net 1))
 (segment (start 114.0178 105.7747) (end 114.0178 94.8078) (width 1.016) (layer B.Cu) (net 1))
 (segment (start 114.0178 94.8078) (end 110.911 91.701) (width 1.016) (layer B.Cu) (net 1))
 (segment (start 177.3314 122.301) (end 178.8041 122.301) (width 1.016) (layer B.Cu) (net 1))
 (segment (start 178.8041 122.301) (end 179.451 122.9479) (width 1.016) (layer B.Cu) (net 1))
 (segment (start 170.561 122.301) (end 177.3314 122.301) (width 1.016) (layer B.Cu) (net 1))
 (segment (start 177.3314 122.301) (end 177.3314 113.6137) (width 1.016) (layer B.Cu) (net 1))
 (segment (start 177.3314 113.6137) (end 179.451 111.4941) (width 1.016) (layer B.Cu) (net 1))
 (segment (start 179.451 109.601) (end 179.451 111.4941) (width 1.016) (layer B.Cu) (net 1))
 (segment (start 121.031 129.921) (end 121.031 128.0279) (width 1.016) (layer B.Cu) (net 1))
 (segment (start 121.031 128.0279) (end 126.7579 122.301) (width 1.016) (layer B.Cu) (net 1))
 (segment (start 126.7579 122.301) (end 129.921 122.301) (width 1.016) (layer B.Cu) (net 1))
 (segment (start 179.451 124.841) (end 179.451 122.9479) (width 1.016) (layer B.Cu) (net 1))
 (segment (start 170.561 118.491) (end 170.561 122.301) (width 1.016) (layer B.Cu) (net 1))
 (segment (start 121.031 114.681) (end 121.031 116.5741) (width 1.016) (layer F.Cu) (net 1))
 (segment (start 129.921 118.491) (end 122.9479 118.491) (width 1.016) (layer F.Cu) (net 1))
 (segment (start 122.9479 118.491) (end 121.031 116.5741) (width 1.016) (layer F.Cu) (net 1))
 (segment (start 129.921 118.491) (end 129.921 122.301) (width 1.016) (layer B.Cu) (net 1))
 (segment (start 192.0278 84.201) (end 192.0278 93.391) (width 1.016) (layer B.Cu) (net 1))
 (segment (start 192.0278 93.391) (end 179.451 105.9678) (width 1.016) (layer B.Cu) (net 1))
 (segment (start 179.451 105.9678) (end 179.451 109.601) (width 1.016) (layer B.Cu) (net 1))
 (segment (start 186.944 77.201) (end 186.944 79.1172) (width 1.016) (layer B.Cu) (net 1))
 (segment (start 186.944 79.1172) (end 192.0278 84.201) (width 1.016) (layer B.Cu) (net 1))
 (segment (start 193.544 84.201) (end 192.0278 84.201) (width 1.016) (layer B.Cu) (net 1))
 (segment (start 173.101 75.311) (end 169.291 75.311) (width 1.016) (layer B.Cu) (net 1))
 (segment (start 142.621 67.691) (end 144.7641 67.691) (width 1.016) (layer F.Cu) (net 1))
 (segment (start 144.7641 67.691) (end 146.9632 65.4919) (width 1.016) (layer F.Cu) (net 1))
 (segment (start 146.9632 65.4919) (end 158.6969 65.4919) (width 1.016) (layer F.Cu) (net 1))
 (segment (start 158.6969 65.4919) (end 168.516 75.311) (width 1.016) (layer F.Cu) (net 1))
 (segment (start 168.516 75.311) (end 169.291 75.311) (width 1.016) (layer F.Cu) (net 1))
 (segment (start 142.621 67.691) (end 137.541 67.691) (width 1.016) (layer F.Cu) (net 1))
 (segment (start 128.0755 79.121) (end 129.921 79.121) (width 1.016) (layer F.Cu) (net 1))
 (segment (start 120.011 84.201) (end 125.091 79.121) (width 1.016) (layer F.Cu) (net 1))
 (segment (start 125.091 79.121) (end 128.0755 79.121) (width 1.016) (layer F.Cu) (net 1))
 (segment (start 137.541 67.691) (end 136.1963 67.691) (width 1.016) (layer F.Cu) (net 1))
 (segment (start 136.1963 67.691) (end 128.0755 75.8118) (width 1.016) (layer F.Cu) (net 1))
 (segment (start 128.0755 75.8118) (end 128.0755 79.121) (width 1.016) (layer F.Cu) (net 1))
 (segment (start 113.411 84.201) (end 120.011 84.201) (width 1.016) (layer F.Cu) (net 1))
 (segment (start 107.211 84.201) (end 113.411 84.201) (width 1.016) (layer F.Cu) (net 1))
 (segment (start 113.411 77.201) (end 113.411 84.201) (width 1.016) (layer F.Cu) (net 1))
 (segment (start 107.211 84.201) (end 110.911 87.901) (width 1.016) (layer B.Cu) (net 1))
 (segment (start 110.911 87.901) (end 110.911 91.701) (width 1.016) (layer B.Cu) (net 1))
 (segment (start 180.744 84.201) (end 180.744 82.954) (width 1.016) (layer F.Cu) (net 1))
 (segment (start 180.744 82.954) (end 173.101 75.311) (width 1.016) (layer F.Cu) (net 1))
 (segment (start 193.544 84.201) (end 180.744 84.201) (width 1.016) (layer F.Cu) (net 1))
 (segment (start 180.744 84.201) (end 180.744 88.001) (width 1.016) (layer B.Cu) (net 1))
 (segment (start 180.744 88.001) (end 184.444 91.701) (width 1.016) (layer B.Cu) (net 1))
 (segment (start 157.861 118.491) (end 157.861 113.411) (width 1.016) (layer B.Cu) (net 10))
 (segment (start 157.861 128.651) (end 156.591 128.651) (width 1.016) (layer B.Cu) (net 8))
 (segment (start 156.591 128.651) (end 155.321 127.381) (width 1.016) (layer B.Cu) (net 8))
 (segment (start 155.321 127.381) (end 155.321 123.571) (width 1.016) (layer B.Cu) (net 8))
 (segment (start 155.321 123.571) (end 156.591 122.301) (width 1.016) (layer B.Cu) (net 8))
 (segment (start 156.591 122.301) (end 157.861 122.301) (width 1.016) (layer B.Cu) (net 8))
 (segment (start 142.621 128.651) (end 143.891 128.651) (width 1.016) (layer B.Cu) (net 9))
 (segment (start 143.891 128.651) (end 145.161 127.381) (width 1.016) (layer B.Cu) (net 9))
 (segment (start 145.161 127.381) (end 145.161 123.571) (width 1.016) (layer B.Cu) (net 9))
 (segment (start 145.161 123.571) (end 143.891 122.301) (width 1.016) (layer B.Cu) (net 9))
 (segment (start 143.891 122.301) (end 142.621 122.301) (width 1.016) (layer B.Cu) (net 9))
 (segment (start 142.621 113.411) (end 142.621 118.491) (width 1.016) (layer B.Cu) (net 11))
 (segment (start 189.571 77.201) (end 189.444 77.201) (width 1.016) (layer B.Cu) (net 6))
 (segment (start 189.571 77.201) (end 190.261 77.201) (width 1.016) (layer B.Cu) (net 6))
 (segment (start 190.261 77.201) (end 192.151 75.311) (width 1.016) (layer B.Cu) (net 6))
 (segment (start 192.151 75.311) (end 192.151 71.501) (width 1.016) (layer B.Cu) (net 6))
 (segment (start 192.151 71.501) (end 189.611 68.961) (width 1.016) (layer B.Cu) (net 6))
 (segment (start 189.611 68.961) (end 189.611 65.151) (width 1.016) (layer B.Cu) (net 6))
 (segment (start 114.681 81.661) (end 114.681 80.391) (width 1.016) (layer B.Cu) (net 15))
 (segment (start 133.731 86.741) (end 132.461 86.741) (width 1.016) (layer B.Cu) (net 15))
 (segment (start 132.461 86.741) (end 129.921 89.281) (width 1.016) (layer B.Cu) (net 15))
 (segment (start 129.921 89.281) (end 118.491 89.281) (width 1.016) (layer B.Cu) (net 15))
 (segment (start 118.491 89.281) (end 114.681 85.471) (width 1.016) (layer B.Cu) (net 15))
 (segment (start 114.681 85.471) (end 114.681 81.661) (width 1.016) (layer B.Cu) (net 15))
 (segment (start 115.911 77.201) (end 115.911 79.161) (width 1.016) (layer B.Cu) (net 15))
 (segment (start 115.911 79.161) (end 114.681 80.391) (width 1.016) (layer B.Cu) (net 15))
 (segment (start 114.681 80.391) (end 113.411 80.391) (width 1.016) (layer B.Cu) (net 15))
 (segment (start 113.411 80.391) (end 108.331 80.391) (width 1.016) (layer B.Cu) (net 15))
 (segment (start 108.331 80.391) (end 107.061 79.121) (width 1.016) (layer B.Cu) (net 15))
 (segment (start 107.061 79.121) (end 107.061 66.421) (width 1.016) (layer B.Cu) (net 15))
 (segment (start 107.061 66.421) (end 108.331 65.151) (width 1.016) (layer B.Cu) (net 15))
 (segment (start 108.331 65.151) (end 110.871 65.151) (width 1.016) (layer B.Cu) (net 15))
 (segment (start 114.681 81.661) (end 113.411 80.391) (width 1.016) (layer B.Cu) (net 15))
 (segment (start 110.871 72.771) (end 110.911 72.811) (width 1.016) (layer B.Cu) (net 17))
 (segment (start 110.911 72.811) (end 110.911 77.201) (width 1.016) (layer B.Cu) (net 17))
 (segment (start 110.871 68.961) (end 110.871 72.771) (width 1.016) (layer B.Cu) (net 17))
 (segment (start 184.571 76.541) (end 184.444 76.668) (width 1.016) (layer B.Cu) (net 13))
 (segment (start 184.444 76.668) (end 184.444 77.201) (width 1.016) (layer B.Cu) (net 13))
 (segment (start 184.571 76.541) (end 184.571 75.271) (width 1.016) (layer B.Cu) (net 13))
 (segment (start 184.571 75.271) (end 187.071 72.771) (width 1.016) (layer B.Cu) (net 13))
 (segment (start 187.071 72.771) (end 189.611 72.771) (width 1.016) (layer B.Cu) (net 13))
 (segment (start 164.211 80.391) (end 181.991 80.391) (width 1.016) (layer B.Cu) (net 13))
 (segment (start 181.991 80.391) (end 184.571 77.811) (width 1.016) (layer B.Cu) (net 13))
 (segment (start 184.571 77.811) (end 184.571 76.541) (width 1.016) (layer B.Cu) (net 13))
 (segment (start 123.571 65.151) (end 123.571 68.961) (width 1.016) (layer B.Cu) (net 12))
 (segment (start 157.861 72.771) (end 155.321 72.771) (width 1.016) (layer B.Cu) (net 12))
 (segment (start 155.321 72.771) (end 147.701 65.151) (width 1.016) (layer B.Cu) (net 12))
 (segment (start 147.701 65.151) (end 123.571 65.151) (width 1.016) (layer B.Cu) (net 12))
 (segment (start 157.861 72.771) (end 160.401 72.771) (width 1.016) (layer B.Cu) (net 12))
 (segment (start 160.401 72.771) (end 164.211 68.961) (width 1.016) (layer B.Cu) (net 12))
 (segment (start 164.211 68.961) (end 164.211 67.691) (width 1.016) (layer B.Cu) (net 12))
 (segment (start 164.211 67.691) (end 164.211 66.421) (width 1.016) (layer B.Cu) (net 12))
 (segment (start 164.211 66.421) (end 165.481 65.151) (width 1.016) (layer B.Cu) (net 12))
 (segment (start 165.481 65.151) (end 176.911 65.151) (width 1.016) (layer B.Cu) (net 12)))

